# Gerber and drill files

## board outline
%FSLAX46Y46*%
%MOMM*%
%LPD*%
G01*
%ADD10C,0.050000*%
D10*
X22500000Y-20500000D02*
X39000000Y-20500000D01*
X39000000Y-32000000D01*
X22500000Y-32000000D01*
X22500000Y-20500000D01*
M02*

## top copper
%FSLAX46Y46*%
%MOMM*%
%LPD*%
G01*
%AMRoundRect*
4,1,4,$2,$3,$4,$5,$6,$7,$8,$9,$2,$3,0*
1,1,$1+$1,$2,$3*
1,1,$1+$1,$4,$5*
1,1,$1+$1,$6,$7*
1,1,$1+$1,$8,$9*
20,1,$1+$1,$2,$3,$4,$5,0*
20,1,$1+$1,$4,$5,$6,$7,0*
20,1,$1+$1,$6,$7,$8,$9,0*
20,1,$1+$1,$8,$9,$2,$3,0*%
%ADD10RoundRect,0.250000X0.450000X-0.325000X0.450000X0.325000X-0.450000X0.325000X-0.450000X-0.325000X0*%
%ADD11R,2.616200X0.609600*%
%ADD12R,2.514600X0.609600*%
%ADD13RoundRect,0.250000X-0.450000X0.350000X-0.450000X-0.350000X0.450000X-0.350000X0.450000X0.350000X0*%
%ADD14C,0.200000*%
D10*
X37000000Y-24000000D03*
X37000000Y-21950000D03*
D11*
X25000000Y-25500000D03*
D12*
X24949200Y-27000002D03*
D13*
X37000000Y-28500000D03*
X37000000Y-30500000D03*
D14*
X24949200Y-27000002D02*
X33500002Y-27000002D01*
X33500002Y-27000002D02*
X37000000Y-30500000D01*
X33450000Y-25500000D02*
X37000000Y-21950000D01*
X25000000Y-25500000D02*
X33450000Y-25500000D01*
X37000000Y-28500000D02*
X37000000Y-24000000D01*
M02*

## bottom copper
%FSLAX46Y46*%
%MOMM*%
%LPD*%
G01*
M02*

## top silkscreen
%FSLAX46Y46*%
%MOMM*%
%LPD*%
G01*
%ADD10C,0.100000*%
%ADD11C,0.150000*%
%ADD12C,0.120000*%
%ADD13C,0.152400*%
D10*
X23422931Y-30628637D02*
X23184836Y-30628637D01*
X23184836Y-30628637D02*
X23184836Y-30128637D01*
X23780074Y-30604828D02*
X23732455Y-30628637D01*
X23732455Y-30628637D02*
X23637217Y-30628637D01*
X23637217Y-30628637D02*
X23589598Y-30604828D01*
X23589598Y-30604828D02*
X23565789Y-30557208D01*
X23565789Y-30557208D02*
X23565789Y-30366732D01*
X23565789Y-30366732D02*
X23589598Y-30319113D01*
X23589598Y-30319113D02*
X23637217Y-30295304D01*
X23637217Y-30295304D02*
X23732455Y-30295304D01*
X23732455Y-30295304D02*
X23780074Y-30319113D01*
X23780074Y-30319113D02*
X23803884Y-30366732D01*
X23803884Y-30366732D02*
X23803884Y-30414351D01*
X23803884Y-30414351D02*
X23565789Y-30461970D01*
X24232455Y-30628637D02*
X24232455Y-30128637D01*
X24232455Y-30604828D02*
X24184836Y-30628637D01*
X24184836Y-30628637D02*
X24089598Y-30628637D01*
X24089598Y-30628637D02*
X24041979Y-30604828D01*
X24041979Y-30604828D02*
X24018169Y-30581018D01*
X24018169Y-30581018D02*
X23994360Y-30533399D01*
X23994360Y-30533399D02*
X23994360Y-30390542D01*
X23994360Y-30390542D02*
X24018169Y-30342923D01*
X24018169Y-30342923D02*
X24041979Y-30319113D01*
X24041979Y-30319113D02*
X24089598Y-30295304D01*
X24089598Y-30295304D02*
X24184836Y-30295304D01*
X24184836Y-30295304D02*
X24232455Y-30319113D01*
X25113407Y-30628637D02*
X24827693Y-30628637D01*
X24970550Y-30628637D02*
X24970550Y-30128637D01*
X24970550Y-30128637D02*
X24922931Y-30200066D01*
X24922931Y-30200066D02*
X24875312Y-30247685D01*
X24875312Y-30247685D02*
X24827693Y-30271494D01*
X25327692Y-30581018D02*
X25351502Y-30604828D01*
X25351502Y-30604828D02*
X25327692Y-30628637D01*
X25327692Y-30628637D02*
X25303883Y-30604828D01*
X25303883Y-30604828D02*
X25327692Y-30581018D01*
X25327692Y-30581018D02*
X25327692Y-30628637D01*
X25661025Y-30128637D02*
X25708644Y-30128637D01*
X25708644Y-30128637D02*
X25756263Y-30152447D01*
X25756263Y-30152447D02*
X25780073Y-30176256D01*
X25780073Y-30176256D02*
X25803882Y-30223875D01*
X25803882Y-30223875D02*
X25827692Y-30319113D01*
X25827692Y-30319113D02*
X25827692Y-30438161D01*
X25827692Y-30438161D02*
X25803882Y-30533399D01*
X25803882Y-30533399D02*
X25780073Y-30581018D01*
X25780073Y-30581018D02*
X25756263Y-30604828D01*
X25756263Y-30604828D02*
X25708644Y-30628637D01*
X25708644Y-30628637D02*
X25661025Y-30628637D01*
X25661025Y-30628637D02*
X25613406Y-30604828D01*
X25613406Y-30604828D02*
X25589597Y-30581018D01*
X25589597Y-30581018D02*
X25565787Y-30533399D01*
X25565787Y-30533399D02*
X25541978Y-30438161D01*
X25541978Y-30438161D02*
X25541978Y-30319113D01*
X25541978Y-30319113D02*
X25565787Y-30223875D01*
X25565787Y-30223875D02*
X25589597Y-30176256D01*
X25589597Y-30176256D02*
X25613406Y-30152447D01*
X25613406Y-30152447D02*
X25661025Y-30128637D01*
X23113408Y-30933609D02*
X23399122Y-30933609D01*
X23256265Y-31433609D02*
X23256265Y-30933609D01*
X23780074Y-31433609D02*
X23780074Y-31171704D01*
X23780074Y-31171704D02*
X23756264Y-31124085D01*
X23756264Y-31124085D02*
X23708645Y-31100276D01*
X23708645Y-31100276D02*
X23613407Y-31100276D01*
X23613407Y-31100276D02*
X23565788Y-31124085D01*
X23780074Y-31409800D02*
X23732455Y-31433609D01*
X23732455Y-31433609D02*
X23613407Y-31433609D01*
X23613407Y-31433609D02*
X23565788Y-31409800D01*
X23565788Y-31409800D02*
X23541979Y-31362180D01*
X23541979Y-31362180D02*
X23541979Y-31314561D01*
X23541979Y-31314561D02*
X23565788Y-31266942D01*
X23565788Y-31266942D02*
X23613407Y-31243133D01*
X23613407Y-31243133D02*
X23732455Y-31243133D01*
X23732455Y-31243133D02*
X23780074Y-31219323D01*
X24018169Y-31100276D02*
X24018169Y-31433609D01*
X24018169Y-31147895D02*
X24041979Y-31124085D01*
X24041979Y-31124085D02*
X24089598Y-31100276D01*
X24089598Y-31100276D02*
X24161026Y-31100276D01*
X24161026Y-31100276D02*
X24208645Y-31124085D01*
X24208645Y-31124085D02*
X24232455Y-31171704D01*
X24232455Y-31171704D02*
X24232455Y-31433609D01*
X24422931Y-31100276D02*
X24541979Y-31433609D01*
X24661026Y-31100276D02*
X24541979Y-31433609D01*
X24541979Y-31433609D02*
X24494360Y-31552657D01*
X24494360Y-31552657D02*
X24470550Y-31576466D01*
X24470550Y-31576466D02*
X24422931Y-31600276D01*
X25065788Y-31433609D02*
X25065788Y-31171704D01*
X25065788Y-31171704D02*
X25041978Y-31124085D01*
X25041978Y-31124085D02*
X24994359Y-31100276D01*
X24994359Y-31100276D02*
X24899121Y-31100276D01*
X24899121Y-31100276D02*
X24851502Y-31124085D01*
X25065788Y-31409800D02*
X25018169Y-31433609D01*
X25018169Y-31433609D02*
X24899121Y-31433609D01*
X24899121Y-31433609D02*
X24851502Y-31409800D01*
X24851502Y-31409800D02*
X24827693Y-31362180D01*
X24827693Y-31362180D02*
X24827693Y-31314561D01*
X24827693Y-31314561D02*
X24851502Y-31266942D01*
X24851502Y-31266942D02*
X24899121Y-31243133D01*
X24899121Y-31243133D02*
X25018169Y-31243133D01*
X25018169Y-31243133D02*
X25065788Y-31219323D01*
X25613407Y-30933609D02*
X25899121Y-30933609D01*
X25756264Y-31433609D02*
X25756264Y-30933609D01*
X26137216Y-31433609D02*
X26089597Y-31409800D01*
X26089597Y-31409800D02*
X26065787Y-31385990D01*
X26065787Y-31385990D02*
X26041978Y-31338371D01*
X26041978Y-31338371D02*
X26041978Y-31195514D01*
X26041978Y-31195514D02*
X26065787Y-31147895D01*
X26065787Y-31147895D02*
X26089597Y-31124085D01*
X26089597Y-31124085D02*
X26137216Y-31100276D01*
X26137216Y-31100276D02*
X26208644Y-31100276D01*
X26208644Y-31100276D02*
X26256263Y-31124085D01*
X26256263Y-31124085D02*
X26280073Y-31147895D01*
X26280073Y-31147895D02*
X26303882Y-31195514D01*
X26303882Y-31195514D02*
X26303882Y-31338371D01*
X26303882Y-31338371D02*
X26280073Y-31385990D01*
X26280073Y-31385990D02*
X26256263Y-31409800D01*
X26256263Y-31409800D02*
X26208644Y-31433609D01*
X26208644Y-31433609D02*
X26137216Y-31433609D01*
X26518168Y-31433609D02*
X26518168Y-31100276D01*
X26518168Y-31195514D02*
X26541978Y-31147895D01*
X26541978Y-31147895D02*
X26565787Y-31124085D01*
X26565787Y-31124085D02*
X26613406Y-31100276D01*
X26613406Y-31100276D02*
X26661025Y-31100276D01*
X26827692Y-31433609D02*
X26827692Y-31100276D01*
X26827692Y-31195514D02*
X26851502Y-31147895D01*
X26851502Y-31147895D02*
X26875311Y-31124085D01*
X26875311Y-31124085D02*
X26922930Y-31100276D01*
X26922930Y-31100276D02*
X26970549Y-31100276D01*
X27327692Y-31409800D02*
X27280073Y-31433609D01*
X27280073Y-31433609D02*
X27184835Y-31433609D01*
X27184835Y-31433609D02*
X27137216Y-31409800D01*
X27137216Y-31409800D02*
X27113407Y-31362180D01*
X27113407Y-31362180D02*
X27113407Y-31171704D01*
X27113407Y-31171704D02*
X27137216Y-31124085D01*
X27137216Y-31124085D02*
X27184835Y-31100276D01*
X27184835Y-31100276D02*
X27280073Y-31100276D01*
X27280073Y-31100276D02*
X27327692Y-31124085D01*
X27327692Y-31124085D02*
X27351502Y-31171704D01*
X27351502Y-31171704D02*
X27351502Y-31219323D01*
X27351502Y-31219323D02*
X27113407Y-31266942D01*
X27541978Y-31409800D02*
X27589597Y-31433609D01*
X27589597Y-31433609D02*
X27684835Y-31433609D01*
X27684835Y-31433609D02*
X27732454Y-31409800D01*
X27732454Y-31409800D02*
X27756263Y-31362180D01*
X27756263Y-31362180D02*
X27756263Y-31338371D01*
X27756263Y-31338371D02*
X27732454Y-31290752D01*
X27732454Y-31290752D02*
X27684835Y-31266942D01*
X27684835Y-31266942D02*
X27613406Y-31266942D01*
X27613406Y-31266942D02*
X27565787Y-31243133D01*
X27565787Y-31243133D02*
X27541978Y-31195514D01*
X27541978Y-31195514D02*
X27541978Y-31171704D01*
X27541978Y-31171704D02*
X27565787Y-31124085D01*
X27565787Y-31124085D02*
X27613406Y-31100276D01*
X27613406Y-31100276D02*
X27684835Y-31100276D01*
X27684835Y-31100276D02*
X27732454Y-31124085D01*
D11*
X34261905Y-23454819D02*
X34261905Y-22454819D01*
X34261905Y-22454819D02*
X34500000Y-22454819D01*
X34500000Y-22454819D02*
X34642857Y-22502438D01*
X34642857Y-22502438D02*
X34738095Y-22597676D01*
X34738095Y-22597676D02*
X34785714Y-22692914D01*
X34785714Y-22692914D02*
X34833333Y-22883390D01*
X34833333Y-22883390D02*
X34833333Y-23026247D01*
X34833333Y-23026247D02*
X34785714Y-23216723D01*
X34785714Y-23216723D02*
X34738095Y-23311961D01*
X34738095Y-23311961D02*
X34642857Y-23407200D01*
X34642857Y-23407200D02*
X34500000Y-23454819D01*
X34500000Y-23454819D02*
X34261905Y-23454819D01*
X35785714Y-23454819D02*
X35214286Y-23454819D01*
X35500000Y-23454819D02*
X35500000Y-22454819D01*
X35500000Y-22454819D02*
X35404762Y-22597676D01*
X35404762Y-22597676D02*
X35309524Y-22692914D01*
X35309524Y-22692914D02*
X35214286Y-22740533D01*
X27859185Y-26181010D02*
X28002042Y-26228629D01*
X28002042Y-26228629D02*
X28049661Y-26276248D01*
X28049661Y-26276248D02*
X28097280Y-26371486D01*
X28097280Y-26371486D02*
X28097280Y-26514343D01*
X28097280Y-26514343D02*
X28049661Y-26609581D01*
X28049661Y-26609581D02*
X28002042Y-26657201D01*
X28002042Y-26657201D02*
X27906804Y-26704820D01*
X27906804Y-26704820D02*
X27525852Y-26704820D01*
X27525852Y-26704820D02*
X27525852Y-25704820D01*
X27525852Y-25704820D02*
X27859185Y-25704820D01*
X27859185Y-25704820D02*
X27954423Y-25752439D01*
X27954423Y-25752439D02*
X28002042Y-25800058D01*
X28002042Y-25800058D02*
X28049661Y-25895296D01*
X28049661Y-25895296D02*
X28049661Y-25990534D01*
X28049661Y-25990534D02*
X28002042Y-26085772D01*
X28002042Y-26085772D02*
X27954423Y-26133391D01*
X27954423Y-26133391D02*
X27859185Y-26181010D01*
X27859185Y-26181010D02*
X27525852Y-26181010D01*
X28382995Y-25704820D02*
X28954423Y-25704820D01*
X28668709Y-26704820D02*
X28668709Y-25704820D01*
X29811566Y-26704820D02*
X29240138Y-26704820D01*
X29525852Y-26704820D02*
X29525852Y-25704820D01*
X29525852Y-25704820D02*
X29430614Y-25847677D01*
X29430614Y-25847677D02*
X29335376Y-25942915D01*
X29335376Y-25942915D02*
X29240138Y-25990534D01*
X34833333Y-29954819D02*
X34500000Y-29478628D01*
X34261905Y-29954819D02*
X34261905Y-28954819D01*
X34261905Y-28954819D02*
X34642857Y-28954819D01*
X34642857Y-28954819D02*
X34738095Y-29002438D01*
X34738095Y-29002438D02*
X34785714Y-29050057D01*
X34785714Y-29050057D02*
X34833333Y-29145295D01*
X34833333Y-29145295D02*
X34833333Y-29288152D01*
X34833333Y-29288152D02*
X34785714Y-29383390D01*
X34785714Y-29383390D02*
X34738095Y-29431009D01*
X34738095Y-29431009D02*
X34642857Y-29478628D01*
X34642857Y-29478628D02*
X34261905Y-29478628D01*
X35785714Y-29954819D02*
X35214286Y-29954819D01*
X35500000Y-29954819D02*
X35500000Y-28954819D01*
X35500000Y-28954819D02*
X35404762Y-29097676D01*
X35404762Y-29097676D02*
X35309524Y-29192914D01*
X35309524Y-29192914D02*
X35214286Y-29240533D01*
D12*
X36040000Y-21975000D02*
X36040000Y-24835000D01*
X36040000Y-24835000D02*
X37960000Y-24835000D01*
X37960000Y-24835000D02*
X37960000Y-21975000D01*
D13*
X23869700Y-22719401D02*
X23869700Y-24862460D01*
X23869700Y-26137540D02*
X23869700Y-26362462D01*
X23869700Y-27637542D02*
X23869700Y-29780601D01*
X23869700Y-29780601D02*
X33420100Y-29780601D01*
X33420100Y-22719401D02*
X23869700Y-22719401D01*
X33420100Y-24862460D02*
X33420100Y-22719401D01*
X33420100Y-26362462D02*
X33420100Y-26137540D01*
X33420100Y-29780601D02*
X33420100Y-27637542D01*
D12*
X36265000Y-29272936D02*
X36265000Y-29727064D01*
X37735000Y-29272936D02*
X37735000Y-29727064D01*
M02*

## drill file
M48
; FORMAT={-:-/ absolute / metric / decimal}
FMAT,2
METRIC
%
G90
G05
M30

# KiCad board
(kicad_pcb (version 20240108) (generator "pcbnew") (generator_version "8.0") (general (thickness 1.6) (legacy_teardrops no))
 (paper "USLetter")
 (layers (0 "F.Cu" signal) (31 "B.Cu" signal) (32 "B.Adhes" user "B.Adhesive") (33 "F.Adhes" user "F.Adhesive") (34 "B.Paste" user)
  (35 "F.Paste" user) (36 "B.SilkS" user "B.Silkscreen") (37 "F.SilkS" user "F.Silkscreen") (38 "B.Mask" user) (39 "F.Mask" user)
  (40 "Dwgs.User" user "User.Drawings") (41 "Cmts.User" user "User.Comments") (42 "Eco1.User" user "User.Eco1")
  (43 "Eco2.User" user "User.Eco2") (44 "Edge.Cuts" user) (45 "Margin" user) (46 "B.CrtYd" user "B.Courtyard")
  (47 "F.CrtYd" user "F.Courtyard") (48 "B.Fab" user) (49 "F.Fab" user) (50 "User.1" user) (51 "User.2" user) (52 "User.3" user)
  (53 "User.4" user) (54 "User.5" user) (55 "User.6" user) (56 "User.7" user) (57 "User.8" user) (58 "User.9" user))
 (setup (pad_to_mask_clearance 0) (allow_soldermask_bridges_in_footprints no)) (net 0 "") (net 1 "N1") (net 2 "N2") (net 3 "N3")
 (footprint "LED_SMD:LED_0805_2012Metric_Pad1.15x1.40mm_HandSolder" (layer "F.Cu") (at 37 22.975 90)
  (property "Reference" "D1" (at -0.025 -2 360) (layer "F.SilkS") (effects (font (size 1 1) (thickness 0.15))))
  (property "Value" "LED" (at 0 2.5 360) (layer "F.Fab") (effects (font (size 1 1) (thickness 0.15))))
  (fp_line (start 1 -0.96) (end -1.86 -0.96) (stroke (width 0.12) (type solid)) (layer "F.SilkS"))
  (fp_line (start -1.86 -0.96) (end -1.86 0.96) (stroke (width 0.12) (type solid)) (layer "F.SilkS"))
  (fp_line (start -1.86 0.96) (end 1 0.96) (stroke (width 0.12) (type solid)) (layer "F.SilkS"))
  (pad "1" smd roundrect (at -1.025 0 90) (size 1.15 1.4) (layers "F.Cu" "F.Paste" "F.Mask") (roundrect_rratio 0.217391) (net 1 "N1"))
  (pad "2" smd roundrect (at 1.025 0 90) (size 1.15 1.4) (layers "F.Cu" "F.Paste" "F.Mask") (roundrect_rratio 0.217391) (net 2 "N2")))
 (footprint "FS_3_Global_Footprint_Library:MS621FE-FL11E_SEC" (layer "F.Cu") (at 28.6449 26.250001)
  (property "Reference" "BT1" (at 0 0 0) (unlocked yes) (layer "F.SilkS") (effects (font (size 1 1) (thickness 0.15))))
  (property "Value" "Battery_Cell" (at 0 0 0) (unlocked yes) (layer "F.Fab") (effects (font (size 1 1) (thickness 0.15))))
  (fp_line (start -4.7752 -3.5306) (end -4.7752 -1.387541) (stroke (width 0.1524) (type solid)) (layer "F.SilkS"))
  (fp_line (start -4.7752 -0.112461) (end -4.7752 0.112461) (stroke (width 0.1524) (type solid)) (layer "F.SilkS"))
  (fp_line (start -4.7752 1.387541) (end -4.7752 3.5306) (stroke (width 0.1524) (type solid)) (layer "F.SilkS"))
  (fp_line (start -4.7752 3.5306) (end 4.7752 3.5306) (stroke (width 0.1524) (type solid)) (layer "F.SilkS"))
  (fp_line (start 4.7752 -3.5306) (end -4.7752 -3.5306) (stroke (width 0.1524) (type solid)) (layer "F.SilkS"))
  (fp_line (start 4.7752 -1.387541) (end 4.7752 -3.5306) (stroke (width 0.1524) (type solid)) (layer "F.SilkS"))
  (fp_line (start 4.7752 0.112461) (end 4.7752 -0.112461) (stroke (width 0.1524) (type solid)) (layer "F.SilkS"))
  (fp_line (start 4.7752 3.5306) (end 4.7752 1.387541) (stroke (width 0.1524) (type solid)) (layer "F.SilkS"))
  (pad "1" smd rect (at -3.6449 -0.750001) (size 2.6162 0.6096) (layers "F.Cu" "F.Paste" "F.Mask") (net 2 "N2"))
  (pad "2" smd rect (at -3.6957 0.750001) (size 2.5146 0.6096) (layers "F.Cu" "F.Paste" "F.Mask") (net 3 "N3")))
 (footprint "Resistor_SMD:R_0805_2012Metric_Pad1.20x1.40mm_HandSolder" (layer "F.Cu") (at 37 29.5 -90)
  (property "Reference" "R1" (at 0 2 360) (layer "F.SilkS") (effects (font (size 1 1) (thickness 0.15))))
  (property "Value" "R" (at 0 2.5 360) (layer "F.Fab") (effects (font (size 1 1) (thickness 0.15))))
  (fp_line (start -0.227064 0.735) (end 0.227064 0.735) (stroke (width 0.12) (type solid)) (layer "F.SilkS"))
  (fp_line (start -0.227064 -0.735) (end 0.227064 -0.735) (stroke (width 0.12) (type solid)) (layer "F.SilkS"))
  (pad "1" smd roundrect (at -1 0 270) (size 1.2 1.4) (layers "F.Cu" "F.Paste" "F.Mask") (roundrect_rratio 0.208333) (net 1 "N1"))
  (pad "2" smd roundrect (at 1 0 270) (size 1.2 1.4) (layers "F.Cu" "F.Paste" "F.Mask") (roundrect_rratio 0.208333) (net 3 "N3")))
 (gr_rect (start 22.5 20.5) (end 39 32) (stroke (width 0.05) (type default)) (fill none) (layer "Edge.Cuts"))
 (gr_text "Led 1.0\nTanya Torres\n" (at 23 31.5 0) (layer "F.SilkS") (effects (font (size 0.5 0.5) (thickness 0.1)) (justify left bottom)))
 (segment (start 24.9492 27.000002) (end 33.500002 27.000002) (width 0.2) (layer "F.Cu") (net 3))
 (segment (start 33.500002 27.000002) (end 37 30.5) (width 0.2) (layer "F.Cu") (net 3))
 (segment (start 33.45 25.5) (end 37 21.95) (width 0.2) (layer "F.Cu") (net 2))
 (segment (start 25 25.5) (end 33.45 25.5) (width 0.2) (layer "F.Cu") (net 2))
 (segment (start 37 28.5) (end 37 24) (width 0.2) (layer "F.Cu") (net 1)))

